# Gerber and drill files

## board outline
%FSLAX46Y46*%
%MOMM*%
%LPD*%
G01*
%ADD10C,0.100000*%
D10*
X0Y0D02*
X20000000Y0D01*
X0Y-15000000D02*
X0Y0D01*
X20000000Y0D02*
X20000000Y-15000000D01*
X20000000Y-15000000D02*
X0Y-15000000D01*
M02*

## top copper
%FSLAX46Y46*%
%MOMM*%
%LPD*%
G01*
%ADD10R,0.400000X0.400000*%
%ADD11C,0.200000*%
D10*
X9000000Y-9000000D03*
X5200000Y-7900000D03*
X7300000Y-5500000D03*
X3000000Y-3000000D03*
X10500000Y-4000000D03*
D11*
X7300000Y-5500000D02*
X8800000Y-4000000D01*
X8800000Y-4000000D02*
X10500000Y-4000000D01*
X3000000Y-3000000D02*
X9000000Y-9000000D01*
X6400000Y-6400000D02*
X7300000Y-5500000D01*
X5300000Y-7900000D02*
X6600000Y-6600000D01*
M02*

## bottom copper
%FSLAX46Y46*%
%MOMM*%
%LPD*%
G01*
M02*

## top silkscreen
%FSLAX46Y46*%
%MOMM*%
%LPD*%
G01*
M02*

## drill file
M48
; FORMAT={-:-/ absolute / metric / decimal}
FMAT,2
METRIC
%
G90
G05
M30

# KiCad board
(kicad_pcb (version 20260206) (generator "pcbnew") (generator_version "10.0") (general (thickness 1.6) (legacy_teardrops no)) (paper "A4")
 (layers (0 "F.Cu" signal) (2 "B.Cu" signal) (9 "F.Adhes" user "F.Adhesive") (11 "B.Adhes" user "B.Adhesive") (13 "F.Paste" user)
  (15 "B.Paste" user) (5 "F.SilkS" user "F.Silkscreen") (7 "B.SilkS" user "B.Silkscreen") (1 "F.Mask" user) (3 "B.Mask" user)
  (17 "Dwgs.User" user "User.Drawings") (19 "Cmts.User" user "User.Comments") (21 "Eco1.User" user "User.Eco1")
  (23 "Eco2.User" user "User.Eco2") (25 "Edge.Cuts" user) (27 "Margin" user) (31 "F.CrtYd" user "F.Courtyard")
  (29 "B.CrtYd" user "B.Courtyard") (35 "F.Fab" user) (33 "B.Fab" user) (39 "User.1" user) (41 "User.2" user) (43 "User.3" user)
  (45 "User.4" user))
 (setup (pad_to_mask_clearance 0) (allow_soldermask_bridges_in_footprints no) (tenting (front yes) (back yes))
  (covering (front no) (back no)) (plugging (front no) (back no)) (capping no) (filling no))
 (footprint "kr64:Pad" (layer "F.Cu") (at 9 9)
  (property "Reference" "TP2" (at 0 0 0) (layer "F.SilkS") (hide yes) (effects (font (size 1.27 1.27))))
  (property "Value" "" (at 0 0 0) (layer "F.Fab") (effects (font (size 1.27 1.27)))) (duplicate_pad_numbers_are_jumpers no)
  (pad "1" smd rect (at 0 0) (size 0.4 0.4) (layers "F.Cu" "F.Mask" "F.Paste") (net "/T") (thermal_bridge_angle 45)))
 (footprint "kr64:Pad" (layer "F.Cu") (at 5.2 7.9)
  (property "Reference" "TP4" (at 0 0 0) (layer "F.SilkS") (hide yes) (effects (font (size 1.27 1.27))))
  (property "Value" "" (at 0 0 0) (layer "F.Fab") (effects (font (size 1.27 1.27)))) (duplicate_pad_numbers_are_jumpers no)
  (pad "1" smd rect (at 0 0) (size 0.4 0.4) (layers "F.Cu" "F.Mask" "F.Paste") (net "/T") (thermal_bridge_angle 45)))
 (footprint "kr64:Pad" (layer "F.Cu") (at 7.3 5.5)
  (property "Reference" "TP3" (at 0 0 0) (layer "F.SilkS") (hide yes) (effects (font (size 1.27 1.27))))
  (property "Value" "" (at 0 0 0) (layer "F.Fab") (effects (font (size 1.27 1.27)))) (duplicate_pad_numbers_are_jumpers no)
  (pad "1" smd rect (at 0 0) (size 0.4 0.4) (layers "F.Cu" "F.Mask" "F.Paste") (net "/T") (thermal_bridge_angle 45)))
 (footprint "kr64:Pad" (layer "F.Cu") (at 3 3)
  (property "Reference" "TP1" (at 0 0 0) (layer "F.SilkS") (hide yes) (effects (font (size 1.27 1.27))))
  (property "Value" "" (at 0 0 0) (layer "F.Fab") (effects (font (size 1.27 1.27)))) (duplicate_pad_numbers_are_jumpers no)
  (pad "1" smd rect (at 0 0) (size 0.4 0.4) (layers "F.Cu" "F.Mask" "F.Paste") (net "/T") (thermal_bridge_angle 45)))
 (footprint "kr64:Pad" (layer "F.Cu") (at 10.5 4)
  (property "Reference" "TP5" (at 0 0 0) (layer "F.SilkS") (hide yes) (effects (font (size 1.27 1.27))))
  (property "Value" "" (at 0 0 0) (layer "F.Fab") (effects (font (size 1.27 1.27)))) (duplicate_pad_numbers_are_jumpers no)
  (pad "1" smd rect (at 0 0) (size 0.4 0.4) (layers "F.Cu" "F.Mask" "F.Paste") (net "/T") (thermal_bridge_angle 45)))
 (gr_line (start 0 0) (end 20 0) (stroke (width 0.1) (type default)) (layer "Edge.Cuts"))
 (gr_line (start 0 15) (end 0 0) (stroke (width 0.1) (type default)) (layer "Edge.Cuts"))
 (gr_line (start 20 0) (end 20 15) (stroke (width 0.1) (type default)) (layer "Edge.Cuts"))
 (gr_line (start 20 15) (end 0 15) (stroke (width 0.1) (type default)) (layer "Edge.Cuts"))
 (segment (start 7.3 5.5) (end 8.8 4) (width 0.2) (layer "F.Cu") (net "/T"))
 (segment (start 8.8 4) (end 10.5 4) (width 0.2) (layer "F.Cu") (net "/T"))
 (segment (start 3 3) (end 9 9) (width 0.2) (layer "F.Cu") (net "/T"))
 (segment (start 6.4 6.4) (end 7.3 5.5) (width 0.2) (layer "F.Cu") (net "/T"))
 (segment (start 5.3 7.9) (end 6.6 6.6) (width 0.2) (layer "F.Cu") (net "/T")))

